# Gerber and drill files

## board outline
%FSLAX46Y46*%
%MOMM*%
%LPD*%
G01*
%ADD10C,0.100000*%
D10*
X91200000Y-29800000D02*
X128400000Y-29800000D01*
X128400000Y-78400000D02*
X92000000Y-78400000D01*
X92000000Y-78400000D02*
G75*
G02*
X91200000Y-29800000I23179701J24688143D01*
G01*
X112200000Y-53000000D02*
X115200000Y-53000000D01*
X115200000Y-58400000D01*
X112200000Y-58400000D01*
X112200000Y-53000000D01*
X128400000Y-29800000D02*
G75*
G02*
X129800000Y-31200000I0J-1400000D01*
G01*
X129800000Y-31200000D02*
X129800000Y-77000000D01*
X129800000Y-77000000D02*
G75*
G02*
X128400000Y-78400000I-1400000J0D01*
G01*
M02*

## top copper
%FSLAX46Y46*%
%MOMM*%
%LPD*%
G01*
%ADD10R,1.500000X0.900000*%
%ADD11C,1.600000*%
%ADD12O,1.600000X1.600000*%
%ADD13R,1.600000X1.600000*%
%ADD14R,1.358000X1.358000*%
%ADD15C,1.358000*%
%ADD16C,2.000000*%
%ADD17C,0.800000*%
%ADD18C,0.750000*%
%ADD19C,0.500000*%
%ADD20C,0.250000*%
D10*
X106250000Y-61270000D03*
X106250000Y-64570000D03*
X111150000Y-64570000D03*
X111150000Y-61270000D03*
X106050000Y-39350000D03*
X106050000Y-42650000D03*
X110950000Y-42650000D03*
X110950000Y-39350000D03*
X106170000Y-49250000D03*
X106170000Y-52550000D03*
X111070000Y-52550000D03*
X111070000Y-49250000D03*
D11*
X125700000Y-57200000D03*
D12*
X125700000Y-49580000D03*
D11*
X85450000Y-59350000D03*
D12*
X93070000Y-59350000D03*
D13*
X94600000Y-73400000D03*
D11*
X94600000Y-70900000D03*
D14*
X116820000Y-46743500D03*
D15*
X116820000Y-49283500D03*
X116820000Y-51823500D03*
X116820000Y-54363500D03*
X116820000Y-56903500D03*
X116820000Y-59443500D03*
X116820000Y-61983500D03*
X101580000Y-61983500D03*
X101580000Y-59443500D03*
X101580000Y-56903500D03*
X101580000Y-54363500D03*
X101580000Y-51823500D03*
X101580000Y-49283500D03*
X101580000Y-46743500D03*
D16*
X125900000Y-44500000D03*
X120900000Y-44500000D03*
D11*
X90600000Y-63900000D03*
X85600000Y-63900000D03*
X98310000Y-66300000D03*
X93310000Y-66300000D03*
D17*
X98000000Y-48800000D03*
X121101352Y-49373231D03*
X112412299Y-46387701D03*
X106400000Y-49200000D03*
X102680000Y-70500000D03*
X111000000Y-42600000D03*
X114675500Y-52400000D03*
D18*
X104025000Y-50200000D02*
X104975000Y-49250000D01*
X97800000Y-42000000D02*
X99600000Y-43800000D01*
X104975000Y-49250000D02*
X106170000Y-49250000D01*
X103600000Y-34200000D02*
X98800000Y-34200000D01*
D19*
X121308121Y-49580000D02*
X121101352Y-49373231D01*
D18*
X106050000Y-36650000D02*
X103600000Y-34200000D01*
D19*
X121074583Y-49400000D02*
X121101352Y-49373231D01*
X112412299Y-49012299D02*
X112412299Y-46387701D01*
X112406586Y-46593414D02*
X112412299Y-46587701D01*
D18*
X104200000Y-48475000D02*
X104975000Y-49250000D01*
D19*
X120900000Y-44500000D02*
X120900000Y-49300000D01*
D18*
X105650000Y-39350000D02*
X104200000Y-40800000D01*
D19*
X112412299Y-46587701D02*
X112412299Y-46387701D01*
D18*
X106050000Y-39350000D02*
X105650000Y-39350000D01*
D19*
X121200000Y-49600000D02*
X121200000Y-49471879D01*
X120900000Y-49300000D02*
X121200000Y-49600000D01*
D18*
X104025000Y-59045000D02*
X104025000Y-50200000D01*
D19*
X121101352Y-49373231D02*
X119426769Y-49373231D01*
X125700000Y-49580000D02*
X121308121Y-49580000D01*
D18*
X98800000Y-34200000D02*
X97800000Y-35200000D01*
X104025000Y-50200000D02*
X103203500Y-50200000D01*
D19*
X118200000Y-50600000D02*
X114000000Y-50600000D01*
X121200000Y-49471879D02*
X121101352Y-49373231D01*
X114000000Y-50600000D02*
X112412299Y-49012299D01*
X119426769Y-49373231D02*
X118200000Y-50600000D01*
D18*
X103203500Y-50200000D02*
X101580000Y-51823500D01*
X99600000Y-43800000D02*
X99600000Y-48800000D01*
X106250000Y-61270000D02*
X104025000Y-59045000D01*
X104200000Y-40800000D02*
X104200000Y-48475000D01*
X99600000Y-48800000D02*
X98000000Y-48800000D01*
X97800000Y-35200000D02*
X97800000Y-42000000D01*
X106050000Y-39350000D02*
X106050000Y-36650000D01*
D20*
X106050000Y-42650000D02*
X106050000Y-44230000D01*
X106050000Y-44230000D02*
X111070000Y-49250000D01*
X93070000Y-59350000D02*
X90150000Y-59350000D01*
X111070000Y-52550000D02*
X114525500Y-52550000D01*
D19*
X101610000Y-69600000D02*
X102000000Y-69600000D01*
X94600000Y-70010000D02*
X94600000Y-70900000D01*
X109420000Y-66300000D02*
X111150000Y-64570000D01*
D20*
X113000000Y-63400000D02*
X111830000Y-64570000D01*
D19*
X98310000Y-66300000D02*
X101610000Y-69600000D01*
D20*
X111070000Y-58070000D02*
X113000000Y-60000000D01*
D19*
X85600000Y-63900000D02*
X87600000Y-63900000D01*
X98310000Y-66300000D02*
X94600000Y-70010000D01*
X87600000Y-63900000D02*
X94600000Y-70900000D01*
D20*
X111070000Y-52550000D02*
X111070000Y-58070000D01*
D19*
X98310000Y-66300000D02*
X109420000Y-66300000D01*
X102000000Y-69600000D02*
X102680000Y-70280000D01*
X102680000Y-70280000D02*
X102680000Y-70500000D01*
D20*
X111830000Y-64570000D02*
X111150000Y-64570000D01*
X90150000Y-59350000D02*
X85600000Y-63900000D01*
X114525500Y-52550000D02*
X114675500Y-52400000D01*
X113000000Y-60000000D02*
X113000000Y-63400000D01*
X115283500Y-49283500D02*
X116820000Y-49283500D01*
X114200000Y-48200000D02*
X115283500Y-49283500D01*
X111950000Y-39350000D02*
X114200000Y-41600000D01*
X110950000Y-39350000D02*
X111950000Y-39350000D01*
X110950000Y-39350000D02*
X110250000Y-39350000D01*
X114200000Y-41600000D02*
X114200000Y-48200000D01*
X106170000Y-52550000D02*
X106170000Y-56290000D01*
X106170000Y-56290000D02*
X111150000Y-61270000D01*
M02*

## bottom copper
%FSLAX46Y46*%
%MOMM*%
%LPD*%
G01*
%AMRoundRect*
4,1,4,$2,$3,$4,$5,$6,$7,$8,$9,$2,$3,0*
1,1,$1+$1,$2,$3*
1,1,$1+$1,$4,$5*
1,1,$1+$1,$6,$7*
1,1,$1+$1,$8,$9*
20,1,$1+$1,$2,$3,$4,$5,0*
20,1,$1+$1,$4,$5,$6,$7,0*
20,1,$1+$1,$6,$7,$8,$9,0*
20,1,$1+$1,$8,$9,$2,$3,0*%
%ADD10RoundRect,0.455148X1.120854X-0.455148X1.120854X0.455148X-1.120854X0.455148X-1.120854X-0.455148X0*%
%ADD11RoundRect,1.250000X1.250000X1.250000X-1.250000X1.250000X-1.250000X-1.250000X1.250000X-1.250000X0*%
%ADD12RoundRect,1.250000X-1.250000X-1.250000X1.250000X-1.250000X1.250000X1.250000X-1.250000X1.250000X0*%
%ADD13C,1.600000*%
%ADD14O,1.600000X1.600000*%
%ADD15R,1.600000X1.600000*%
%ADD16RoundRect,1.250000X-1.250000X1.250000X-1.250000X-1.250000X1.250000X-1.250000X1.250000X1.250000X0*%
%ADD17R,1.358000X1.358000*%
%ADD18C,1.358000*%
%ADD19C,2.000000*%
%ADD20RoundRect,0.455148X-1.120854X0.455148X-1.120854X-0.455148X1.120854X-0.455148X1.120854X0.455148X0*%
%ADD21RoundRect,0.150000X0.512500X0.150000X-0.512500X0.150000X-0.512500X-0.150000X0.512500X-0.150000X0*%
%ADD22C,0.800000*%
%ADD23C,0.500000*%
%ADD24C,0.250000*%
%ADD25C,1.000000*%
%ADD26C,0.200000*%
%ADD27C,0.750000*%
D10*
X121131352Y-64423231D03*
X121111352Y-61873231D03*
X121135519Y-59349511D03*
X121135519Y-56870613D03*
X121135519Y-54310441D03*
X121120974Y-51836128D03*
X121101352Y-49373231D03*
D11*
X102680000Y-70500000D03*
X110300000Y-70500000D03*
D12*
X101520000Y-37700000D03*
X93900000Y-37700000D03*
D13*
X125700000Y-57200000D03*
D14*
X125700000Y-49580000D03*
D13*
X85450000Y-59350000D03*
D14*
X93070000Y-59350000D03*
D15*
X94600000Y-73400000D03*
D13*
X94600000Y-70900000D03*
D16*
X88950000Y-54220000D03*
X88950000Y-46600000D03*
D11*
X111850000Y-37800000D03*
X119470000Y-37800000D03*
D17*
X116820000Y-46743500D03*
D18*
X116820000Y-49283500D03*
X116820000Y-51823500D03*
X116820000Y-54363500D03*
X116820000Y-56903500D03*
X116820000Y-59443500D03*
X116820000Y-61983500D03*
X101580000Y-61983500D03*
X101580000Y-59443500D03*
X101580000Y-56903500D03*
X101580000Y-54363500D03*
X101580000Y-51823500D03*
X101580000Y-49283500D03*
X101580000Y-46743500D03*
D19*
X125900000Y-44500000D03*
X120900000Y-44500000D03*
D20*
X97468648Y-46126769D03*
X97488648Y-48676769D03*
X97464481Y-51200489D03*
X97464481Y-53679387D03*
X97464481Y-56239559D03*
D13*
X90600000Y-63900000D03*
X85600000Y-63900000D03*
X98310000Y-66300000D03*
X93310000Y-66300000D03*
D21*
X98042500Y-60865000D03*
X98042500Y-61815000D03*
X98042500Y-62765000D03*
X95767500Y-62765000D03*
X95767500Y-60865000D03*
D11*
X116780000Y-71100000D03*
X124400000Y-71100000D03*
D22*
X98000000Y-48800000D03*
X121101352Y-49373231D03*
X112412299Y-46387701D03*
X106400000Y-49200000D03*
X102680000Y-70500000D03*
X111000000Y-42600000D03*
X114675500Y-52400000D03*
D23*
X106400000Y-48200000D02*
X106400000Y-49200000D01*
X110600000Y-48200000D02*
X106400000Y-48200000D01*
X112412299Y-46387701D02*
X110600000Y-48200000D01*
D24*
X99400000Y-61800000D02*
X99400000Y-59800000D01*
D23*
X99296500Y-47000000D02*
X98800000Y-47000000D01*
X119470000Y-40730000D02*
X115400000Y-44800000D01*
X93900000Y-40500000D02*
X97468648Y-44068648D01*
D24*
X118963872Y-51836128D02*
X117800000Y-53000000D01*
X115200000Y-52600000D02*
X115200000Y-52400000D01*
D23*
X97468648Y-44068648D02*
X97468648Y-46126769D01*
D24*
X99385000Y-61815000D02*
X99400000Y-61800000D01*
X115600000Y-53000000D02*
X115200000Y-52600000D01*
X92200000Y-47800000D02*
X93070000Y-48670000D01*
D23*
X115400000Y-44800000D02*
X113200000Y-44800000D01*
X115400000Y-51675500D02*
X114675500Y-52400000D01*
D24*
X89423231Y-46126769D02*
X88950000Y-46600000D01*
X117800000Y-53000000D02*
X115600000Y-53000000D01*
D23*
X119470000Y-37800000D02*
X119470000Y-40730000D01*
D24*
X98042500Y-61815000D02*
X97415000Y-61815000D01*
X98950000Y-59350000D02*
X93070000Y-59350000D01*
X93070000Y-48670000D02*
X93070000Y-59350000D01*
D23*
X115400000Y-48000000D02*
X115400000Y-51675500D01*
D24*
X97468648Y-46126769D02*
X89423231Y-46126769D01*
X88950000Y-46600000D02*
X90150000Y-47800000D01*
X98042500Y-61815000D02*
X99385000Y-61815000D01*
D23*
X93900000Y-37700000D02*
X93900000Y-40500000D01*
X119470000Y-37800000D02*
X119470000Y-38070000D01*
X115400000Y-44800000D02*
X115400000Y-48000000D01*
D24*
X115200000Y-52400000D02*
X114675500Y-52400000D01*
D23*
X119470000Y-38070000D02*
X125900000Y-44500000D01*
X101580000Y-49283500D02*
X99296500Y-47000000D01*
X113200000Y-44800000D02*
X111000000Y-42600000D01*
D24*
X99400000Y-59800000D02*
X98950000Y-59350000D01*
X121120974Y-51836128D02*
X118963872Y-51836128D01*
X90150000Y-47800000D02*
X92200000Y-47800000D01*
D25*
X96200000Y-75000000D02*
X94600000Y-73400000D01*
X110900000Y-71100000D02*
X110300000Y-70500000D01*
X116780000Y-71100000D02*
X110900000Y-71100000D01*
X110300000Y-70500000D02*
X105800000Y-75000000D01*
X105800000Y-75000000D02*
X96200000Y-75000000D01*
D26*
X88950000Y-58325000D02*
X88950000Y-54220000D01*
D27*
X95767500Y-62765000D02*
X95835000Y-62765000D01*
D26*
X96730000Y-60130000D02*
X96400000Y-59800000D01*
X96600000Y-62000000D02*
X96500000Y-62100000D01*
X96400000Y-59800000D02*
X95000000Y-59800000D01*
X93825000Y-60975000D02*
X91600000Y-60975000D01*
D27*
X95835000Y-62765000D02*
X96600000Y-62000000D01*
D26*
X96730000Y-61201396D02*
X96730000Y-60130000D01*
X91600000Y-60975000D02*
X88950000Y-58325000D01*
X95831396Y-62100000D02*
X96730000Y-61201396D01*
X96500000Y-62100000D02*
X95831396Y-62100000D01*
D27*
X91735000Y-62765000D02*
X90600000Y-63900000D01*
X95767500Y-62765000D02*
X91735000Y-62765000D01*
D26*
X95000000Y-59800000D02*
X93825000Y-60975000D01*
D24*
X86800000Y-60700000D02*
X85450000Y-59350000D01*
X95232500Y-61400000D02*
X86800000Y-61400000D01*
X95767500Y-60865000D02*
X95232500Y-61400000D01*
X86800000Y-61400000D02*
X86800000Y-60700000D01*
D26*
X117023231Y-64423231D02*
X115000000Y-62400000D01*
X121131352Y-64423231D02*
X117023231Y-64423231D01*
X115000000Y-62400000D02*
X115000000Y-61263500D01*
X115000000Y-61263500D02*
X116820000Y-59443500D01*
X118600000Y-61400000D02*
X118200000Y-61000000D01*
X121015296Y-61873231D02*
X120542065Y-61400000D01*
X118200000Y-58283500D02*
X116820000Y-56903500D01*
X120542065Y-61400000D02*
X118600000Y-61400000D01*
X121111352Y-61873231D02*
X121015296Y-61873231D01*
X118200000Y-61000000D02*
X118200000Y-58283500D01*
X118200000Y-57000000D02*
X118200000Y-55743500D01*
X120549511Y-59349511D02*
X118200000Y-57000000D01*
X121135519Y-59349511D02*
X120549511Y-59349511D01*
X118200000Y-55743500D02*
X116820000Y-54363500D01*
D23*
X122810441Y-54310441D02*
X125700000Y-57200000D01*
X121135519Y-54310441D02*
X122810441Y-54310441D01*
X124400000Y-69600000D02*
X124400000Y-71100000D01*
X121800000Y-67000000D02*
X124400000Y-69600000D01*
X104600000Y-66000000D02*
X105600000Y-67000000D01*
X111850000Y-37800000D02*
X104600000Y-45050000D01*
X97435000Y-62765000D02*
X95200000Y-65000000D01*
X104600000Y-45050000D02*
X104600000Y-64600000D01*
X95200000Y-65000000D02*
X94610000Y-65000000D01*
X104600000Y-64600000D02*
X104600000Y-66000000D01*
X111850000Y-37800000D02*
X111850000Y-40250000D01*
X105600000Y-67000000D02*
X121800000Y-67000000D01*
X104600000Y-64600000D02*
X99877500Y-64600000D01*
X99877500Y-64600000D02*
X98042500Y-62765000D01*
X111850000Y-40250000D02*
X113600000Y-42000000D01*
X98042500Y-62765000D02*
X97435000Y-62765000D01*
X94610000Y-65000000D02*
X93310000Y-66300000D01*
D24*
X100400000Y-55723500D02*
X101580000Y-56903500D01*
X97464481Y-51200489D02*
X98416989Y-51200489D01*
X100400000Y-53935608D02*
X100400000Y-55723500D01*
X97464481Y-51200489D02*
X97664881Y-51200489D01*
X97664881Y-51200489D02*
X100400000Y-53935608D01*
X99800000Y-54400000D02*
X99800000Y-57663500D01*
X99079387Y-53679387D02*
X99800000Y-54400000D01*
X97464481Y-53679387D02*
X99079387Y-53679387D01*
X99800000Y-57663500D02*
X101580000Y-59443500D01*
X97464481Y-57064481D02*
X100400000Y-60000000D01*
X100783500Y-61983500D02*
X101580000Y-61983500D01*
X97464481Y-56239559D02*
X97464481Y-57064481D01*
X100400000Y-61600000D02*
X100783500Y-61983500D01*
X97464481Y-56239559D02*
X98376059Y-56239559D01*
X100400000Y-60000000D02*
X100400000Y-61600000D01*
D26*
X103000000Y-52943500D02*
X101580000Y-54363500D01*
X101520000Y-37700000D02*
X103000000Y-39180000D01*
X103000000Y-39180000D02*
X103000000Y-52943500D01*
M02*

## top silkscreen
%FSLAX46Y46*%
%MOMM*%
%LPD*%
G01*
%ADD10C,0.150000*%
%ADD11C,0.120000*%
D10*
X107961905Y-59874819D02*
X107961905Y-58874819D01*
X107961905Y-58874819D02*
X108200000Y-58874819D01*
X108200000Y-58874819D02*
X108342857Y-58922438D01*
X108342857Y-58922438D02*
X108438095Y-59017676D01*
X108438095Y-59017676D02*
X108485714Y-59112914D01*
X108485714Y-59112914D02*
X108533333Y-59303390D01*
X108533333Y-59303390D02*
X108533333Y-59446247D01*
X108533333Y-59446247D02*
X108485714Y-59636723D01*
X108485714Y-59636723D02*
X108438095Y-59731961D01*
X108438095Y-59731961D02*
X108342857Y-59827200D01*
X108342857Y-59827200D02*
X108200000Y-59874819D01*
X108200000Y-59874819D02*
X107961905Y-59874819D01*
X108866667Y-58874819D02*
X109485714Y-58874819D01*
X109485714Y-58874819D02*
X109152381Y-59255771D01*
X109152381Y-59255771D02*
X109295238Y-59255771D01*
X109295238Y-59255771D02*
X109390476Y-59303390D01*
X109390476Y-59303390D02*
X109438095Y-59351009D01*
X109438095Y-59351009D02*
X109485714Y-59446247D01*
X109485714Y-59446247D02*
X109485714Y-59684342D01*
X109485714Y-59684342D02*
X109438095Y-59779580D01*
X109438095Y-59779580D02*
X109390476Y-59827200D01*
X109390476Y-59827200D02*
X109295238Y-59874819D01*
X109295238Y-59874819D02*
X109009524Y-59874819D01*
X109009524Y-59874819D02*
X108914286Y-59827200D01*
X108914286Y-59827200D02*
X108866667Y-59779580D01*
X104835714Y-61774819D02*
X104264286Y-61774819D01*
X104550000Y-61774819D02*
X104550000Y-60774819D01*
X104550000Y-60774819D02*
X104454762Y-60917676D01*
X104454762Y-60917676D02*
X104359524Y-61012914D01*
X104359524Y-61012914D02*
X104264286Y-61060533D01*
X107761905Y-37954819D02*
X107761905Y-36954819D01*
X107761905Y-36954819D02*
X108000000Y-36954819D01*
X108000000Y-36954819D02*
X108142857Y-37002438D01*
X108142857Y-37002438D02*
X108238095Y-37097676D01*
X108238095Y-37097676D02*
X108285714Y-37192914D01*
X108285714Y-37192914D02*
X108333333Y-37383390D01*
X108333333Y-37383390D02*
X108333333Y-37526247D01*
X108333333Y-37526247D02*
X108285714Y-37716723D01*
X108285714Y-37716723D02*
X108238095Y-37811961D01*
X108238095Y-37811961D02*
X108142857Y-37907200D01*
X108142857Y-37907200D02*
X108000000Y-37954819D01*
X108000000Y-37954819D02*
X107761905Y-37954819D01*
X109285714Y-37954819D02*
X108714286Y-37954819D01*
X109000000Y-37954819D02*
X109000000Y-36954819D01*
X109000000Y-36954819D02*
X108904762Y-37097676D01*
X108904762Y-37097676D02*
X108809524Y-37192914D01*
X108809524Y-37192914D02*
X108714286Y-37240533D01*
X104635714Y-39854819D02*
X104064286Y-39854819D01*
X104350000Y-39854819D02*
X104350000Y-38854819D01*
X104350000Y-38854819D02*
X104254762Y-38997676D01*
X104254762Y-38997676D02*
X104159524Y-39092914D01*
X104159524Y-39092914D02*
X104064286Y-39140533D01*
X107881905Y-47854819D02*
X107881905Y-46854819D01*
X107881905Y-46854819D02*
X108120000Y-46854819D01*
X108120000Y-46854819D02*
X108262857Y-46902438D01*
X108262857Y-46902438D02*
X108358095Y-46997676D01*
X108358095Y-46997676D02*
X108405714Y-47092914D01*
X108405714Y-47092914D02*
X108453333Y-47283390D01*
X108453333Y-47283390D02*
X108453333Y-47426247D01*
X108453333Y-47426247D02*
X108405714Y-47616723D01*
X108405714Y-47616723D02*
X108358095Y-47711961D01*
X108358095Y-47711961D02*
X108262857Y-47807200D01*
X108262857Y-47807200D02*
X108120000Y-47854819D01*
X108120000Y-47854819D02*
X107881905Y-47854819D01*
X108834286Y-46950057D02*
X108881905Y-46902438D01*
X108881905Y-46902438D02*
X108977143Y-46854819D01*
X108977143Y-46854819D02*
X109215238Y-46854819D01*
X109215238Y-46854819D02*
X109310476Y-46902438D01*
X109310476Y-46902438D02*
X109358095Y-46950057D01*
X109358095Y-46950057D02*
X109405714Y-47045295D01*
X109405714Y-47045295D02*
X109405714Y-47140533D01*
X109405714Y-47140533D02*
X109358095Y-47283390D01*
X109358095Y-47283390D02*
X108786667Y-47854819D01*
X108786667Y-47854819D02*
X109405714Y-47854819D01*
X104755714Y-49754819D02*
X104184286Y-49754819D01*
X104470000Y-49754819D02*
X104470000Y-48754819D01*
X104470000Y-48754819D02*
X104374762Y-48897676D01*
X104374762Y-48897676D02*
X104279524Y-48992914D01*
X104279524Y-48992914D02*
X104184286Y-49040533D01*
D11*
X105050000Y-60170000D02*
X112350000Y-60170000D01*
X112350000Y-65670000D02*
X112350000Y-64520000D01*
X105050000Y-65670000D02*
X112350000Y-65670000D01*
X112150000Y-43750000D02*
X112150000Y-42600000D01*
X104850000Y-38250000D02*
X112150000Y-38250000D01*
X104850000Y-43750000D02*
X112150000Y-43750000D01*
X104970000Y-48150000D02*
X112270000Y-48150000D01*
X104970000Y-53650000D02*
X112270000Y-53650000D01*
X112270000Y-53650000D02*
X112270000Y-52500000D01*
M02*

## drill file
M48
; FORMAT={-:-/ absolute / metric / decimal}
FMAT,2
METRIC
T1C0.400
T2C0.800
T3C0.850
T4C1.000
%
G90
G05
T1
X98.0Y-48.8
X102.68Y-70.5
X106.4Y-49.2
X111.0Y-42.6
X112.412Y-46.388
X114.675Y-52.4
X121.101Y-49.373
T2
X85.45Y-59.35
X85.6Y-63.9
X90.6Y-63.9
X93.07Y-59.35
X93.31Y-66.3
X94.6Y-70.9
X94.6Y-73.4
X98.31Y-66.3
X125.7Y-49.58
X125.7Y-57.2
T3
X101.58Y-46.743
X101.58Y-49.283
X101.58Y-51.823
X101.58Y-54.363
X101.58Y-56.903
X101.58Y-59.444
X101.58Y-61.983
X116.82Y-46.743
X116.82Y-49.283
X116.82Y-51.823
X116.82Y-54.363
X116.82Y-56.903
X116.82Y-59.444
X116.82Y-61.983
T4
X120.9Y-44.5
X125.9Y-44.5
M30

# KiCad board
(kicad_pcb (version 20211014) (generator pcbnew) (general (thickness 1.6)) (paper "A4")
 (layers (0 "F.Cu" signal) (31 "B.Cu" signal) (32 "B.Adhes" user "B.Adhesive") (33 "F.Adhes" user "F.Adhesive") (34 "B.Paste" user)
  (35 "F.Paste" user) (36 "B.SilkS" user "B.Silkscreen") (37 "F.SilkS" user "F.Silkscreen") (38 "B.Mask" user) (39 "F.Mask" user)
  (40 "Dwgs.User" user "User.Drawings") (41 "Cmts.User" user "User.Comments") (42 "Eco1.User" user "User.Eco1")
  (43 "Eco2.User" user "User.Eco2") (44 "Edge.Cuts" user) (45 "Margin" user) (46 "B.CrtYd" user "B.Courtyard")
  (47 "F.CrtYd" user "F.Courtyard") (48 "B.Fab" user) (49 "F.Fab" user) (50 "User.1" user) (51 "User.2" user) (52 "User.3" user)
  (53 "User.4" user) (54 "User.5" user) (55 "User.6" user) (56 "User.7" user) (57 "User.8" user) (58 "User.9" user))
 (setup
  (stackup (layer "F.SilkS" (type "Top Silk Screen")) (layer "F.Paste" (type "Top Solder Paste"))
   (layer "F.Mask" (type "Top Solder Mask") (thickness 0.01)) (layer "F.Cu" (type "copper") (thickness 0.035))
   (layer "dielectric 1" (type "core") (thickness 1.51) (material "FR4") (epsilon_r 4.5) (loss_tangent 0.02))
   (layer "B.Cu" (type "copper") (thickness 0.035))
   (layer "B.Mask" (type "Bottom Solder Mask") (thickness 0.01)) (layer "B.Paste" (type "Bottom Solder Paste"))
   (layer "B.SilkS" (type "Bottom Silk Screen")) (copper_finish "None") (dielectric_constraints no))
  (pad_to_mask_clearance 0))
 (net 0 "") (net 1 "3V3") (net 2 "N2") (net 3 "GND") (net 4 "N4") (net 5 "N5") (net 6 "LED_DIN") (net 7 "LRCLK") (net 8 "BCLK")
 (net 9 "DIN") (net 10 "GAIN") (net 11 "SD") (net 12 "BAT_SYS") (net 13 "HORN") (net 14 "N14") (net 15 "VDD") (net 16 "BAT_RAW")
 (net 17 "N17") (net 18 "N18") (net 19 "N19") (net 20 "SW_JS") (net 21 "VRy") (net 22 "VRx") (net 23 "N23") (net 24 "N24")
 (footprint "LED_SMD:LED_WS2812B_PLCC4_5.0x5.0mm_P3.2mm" (layer "F.Cu") (at 108.7 62.92)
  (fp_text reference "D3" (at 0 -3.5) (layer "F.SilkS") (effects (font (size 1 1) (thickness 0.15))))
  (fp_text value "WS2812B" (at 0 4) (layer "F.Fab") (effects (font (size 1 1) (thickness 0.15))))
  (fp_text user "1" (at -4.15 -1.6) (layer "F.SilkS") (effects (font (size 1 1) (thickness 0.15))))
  (fp_line (start -3.65 -2.75) (end 3.65 -2.75) (layer "F.SilkS") (width 0.12))
  (fp_line (start 3.65 2.75) (end 3.65 1.6) (layer "F.SilkS") (width 0.12))
  (fp_line (start -3.65 2.75) (end 3.65 2.75) (layer "F.SilkS") (width 0.12))
  (pad "1" smd rect (at -2.45 -1.65) (size 1.5 0.9) (layers "F.Cu" "F.Paste" "F.Mask") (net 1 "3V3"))
  (pad "2" smd rect (at -2.45 1.65) (size 1.5 0.9) (layers "F.Cu" "F.Paste" "F.Mask") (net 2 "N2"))
  (pad "3" smd rect (at 2.45 1.65) (size 1.5 0.9) (layers "F.Cu" "F.Paste" "F.Mask") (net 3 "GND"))
  (pad "4" smd rect (at 2.45 -1.65) (size 1.5 0.9) (layers "F.Cu" "F.Paste" "F.Mask") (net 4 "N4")))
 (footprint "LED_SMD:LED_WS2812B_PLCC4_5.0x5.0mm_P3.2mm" (layer "F.Cu") (at 108.5 41)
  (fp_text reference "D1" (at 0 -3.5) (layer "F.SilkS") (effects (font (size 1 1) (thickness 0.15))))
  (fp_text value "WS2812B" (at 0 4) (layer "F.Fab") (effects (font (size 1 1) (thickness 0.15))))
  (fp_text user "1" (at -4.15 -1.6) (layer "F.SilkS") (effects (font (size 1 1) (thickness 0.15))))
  (fp_line (start 3.65 2.75) (end 3.65 1.6) (layer "F.SilkS") (width 0.12))
  (fp_line (start -3.65 -2.75) (end 3.65 -2.75) (layer "F.SilkS") (width 0.12))
  (fp_line (start -3.65 2.75) (end 3.65 2.75) (layer "F.SilkS") (width 0.12))
  (pad "1" smd rect (at -2.45 -1.65) (size 1.5 0.9) (layers "F.Cu" "F.Paste" "F.Mask") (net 1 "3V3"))
  (pad "2" smd rect (at -2.45 1.65) (size 1.5 0.9) (layers "F.Cu" "F.Paste" "F.Mask") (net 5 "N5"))
  (pad "3" smd rect (at 2.45 1.65) (size 1.5 0.9) (layers "F.Cu" "F.Paste" "F.Mask") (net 3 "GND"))
  (pad "4" smd rect (at 2.45 -1.65) (size 1.5 0.9) (layers "F.Cu" "F.Paste" "F.Mask") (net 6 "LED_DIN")))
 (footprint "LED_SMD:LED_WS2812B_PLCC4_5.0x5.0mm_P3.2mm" (layer "F.Cu") (at 108.62 50.9)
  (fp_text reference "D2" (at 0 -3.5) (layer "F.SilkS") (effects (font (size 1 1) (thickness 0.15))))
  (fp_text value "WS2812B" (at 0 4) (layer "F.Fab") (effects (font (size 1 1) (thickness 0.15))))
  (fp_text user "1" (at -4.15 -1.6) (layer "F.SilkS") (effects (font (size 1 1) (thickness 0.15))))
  (fp_line (start -3.65 -2.75) (end 3.65 -2.75) (layer "F.SilkS") (width 0.12))
  (fp_line (start -3.65 2.75) (end 3.65 2.75) (layer "F.SilkS") (width 0.12))
  (fp_line (start 3.65 2.75) (end 3.65 1.6) (layer "F.SilkS") (width 0.12))
  (pad "1" smd rect (at -2.45 -1.65) (size 1.5 0.9) (layers "F.Cu" "F.Paste" "F.Mask") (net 1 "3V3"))
  (pad "2" smd rect (at -2.45 1.65) (size 1.5 0.9) (layers "F.Cu" "F.Paste" "F.Mask") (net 4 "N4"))
  (pad "3" smd rect (at 2.45 1.65) (size 1.5 0.9) (layers "F.Cu" "F.Paste" "F.Mask") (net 3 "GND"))
  (pad "4" smd rect (at 2.45 -1.65) (size 1.5 0.9) (layers "F.Cu" "F.Paste" "F.Mask") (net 5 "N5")))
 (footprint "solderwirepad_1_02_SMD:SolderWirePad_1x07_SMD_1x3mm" (layer "B.Cu") (at 121.1 64.4 90)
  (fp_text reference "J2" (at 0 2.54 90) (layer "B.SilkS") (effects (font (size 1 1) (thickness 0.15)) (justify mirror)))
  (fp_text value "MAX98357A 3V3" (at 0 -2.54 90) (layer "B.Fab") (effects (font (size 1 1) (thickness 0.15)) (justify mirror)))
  (pad "1" smd roundrect (at -0.023231 0.031352 90) (size 1.820592 3.152005) (layers "B.Cu" "B.Paste" "B.Mask") (roundrect_rratio 0.25)
   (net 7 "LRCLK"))
  (pad "2" smd roundrect (at 2.526769 0.011352 90) (size 1.820592 3.152005) (layers "B.Cu" "B.Paste" "B.Mask") (roundrect_rratio 0.25)
   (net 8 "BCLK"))
  (pad "3" smd roundrect (at 5.050489 0.035519 90) (size 1.820592 3.152005) (layers "B.Cu" "B.Paste" "B.Mask") (roundrect_rratio 0.25)
   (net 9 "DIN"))
  (pad "4" smd roundrect (at 7.529387 0.035519 90) (size 1.820592 3.152005) (layers "B.Cu" "B.Paste" "B.Mask") (roundrect_rratio 0.25)
   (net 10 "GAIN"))
  (pad "5" smd roundrect (at 10.089559 0.035519 90) (size 1.820592 3.152005) (layers "B.Cu" "B.Paste" "B.Mask") (roundrect_rratio 0.25)
   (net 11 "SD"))
  (pad "6" smd roundrect (at 12.563872 0.020974 90) (size 1.820592 3.152005) (layers "B.Cu" "B.Paste" "B.Mask") (roundrect_rratio 0.25)
   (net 3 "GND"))
  (pad "7" smd roundrect (at 15.026769 0.001352 90) (size 1.820592 3.152005) (layers "B.Cu" "B.Paste" "B.Mask") (roundrect_rratio 0.25)
   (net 1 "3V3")))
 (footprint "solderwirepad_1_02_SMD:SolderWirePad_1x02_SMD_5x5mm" (layer "B.Cu") (at 110.3 70.5 180)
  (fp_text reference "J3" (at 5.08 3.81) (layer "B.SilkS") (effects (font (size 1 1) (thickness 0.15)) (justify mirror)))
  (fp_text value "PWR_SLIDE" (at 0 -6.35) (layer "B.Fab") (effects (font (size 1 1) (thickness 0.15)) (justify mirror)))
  (pad "1" smd roundrect (at 7.62 0 180) (size 5 5) (layers "B.Cu" "B.Paste" "B.Mask") (roundrect_rratio 0.25) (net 3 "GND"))
  (pad "2" smd roundrect (at 0 0 180) (size 5 5) (layers "B.Cu" "B.Paste" "B.Mask") (roundrect_rratio 0.25) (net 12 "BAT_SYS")))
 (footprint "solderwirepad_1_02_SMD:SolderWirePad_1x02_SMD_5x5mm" (layer "B.Cu") (at 93.9 37.7)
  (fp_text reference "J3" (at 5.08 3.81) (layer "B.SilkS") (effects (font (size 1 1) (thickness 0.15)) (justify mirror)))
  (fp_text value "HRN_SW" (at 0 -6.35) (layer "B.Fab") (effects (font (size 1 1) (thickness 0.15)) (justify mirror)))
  (pad "1" smd roundrect (at 7.62 0) (size 5 5) (layers "B.Cu" "B.Paste" "B.Mask") (roundrect_rratio 0.25) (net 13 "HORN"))
  (pad "2" smd roundrect (at 0 0) (size 5 5) (layers "B.Cu" "B.Paste" "B.Mask") (roundrect_rratio 0.25) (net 3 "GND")))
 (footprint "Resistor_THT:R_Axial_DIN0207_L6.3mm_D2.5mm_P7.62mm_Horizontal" (layer "B.Cu") (at 125.7 57.2 90)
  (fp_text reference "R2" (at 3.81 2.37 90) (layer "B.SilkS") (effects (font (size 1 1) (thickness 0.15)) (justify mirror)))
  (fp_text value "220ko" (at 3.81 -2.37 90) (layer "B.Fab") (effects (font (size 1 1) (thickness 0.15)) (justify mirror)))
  (pad "1" thru_hole circle (at 0 0 90) (size 1.6 1.6) (drill 0.8) (layers *.Cu *.Mask) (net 11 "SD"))
  (pad "2" thru_hole oval (at 7.62 0 90) (size 1.6 1.6) (drill 0.8) (layers *.Cu *.Mask) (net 1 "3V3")))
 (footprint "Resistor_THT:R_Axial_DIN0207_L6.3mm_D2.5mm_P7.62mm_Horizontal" (layer "B.Cu") (at 85.45 59.35)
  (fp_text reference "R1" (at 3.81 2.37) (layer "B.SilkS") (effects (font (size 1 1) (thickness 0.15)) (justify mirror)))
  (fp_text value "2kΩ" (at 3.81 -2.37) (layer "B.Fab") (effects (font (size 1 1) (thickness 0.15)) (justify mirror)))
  (pad "1" thru_hole circle (at 0 0) (size 1.6 1.6) (drill 0.8) (layers *.Cu *.Mask) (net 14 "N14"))
  (pad "2" thru_hole oval (at 7.62 0) (size 1.6 1.6) (drill 0.8) (layers *.Cu *.Mask) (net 3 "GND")))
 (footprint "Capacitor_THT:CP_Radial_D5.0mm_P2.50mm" (layer "B.Cu") (at 94.6 73.4 90)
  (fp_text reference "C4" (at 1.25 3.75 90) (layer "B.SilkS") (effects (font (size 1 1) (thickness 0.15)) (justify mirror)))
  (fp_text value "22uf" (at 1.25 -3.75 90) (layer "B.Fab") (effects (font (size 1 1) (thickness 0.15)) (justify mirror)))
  (pad "1" thru_hole rect (at 0 0 90) (size 1.6 1.6) (drill 0.8) (layers *.Cu *.Mask) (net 12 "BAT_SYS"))
  (pad "2" thru_hole circle (at 2.5 0 90) (size 1.6 1.6) (drill 0.8) (layers *.Cu *.Mask) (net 3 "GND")))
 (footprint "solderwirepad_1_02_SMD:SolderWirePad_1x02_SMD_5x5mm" (layer "B.Cu") (at 88.95 46.6 -90)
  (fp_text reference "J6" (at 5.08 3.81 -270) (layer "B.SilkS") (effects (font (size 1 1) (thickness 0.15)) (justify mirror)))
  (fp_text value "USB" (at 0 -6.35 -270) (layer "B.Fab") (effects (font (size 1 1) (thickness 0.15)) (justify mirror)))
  (pad "1" smd roundrect (at 7.62 0 270) (size 5 5) (layers "B.Cu" "B.Paste" "B.Mask") (roundrect_rratio 0.25) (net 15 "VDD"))
  (pad "2" smd roundrect (at 0 0 270) (size 5 5) (layers "B.Cu" "B.Paste" "B.Mask") (roundrect_rratio 0.25) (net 3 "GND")))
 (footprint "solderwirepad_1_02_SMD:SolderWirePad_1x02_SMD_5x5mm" (layer "B.Cu") (at 119.47 37.8 180)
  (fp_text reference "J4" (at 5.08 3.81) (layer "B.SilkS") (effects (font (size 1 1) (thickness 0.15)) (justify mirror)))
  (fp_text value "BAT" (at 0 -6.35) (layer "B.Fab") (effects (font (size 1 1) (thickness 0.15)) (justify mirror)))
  (pad "1" smd roundrect (at 7.62 0 180) (size 5 5) (layers "B.Cu" "B.Paste" "B.Mask") (roundrect_rratio 0.25) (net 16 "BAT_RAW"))
  (pad "2" smd roundrect (at 0 0 180) (size 5 5) (layers "B.Cu" "B.Paste" "B.Mask") (roundrect_rratio 0.25) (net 3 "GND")))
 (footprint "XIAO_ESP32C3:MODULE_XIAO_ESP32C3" (layer "B.Cu") (at 109.2 54.3 180)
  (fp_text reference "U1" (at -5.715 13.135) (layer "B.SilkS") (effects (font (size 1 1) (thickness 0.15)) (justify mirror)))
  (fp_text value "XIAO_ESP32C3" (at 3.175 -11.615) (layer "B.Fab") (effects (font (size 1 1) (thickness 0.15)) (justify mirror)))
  (pad "1" thru_hole rect (at -7.62 7.5565 180) (size 1.358 1.358) (drill 0.85) (layers *.Cu *.Mask) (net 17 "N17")
   (solder_mask_margin 0.102))
  (pad "2" thru_hole circle (at -7.62 5.0165 180) (size 1.358 1.358) (drill 0.85) (layers *.Cu *.Mask) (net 6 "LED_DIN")
   (solder_mask_margin 0.102))
  (pad "3" thru_hole circle (at -7.62 2.4765 180) (size 1.358 1.358) (drill 0.85) (layers *.Cu *.Mask) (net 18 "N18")
   (solder_mask_margin 0.102))
  (pad "4" thru_hole circle (at -7.62 -0.0635 180) (size 1.358 1.358) (drill 0.85) (layers *.Cu *.Mask) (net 9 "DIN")
   (solder_mask_margin 0.102))
  (pad "5" thru_hole circle (at -7.62 -2.6035 180) (size 1.358 1.358) (drill 0.85) (layers *.Cu *.Mask) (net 8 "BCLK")
   (solder_mask_margin 0.102))
  (pad "6" thru_hole circle (at -7.62 -5.1435 180) (size 1.358 1.358) (drill 0.85) (layers *.Cu *.Mask) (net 7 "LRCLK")
   (solder_mask_margin 0.102))
  (pad "7" thru_hole circle (at -7.62 -7.6835 180) (size 1.358 1.358) (drill 0.85) (layers *.Cu *.Mask) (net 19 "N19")
   (solder_mask_margin 0.102))
  (pad "8" thru_hole circle (at 7.62 -7.6835 180) (size 1.358 1.358) (drill 0.85) (layers *.Cu *.Mask) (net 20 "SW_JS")
   (solder_mask_margin 0.102))
  (pad "9" thru_hole circle (at 7.62 -5.1435 180) (size 1.358 1.358) (drill 0.85) (layers *.Cu *.Mask) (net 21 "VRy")
   (solder_mask_margin 0.102))
  (pad "10" thru_hole circle (at 7.62 -2.6035 180) (size 1.358 1.358) (drill 0.85) (layers *.Cu *.Mask) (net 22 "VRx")
   (solder_mask_margin 0.102))
  (pad "11" thru_hole circle (at 7.62 -0.0635 180) (size 1.358 1.358) (drill 0.85) (layers *.Cu *.Mask) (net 13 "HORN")
   (solder_mask_margin 0.102))
  (pad "12" thru_hole circle (at 7.62 2.4765 180) (size 1.358 1.358) (drill 0.85) (layers *.Cu *.Mask) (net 1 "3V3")
   (solder_mask_margin 0.102))
  (pad "13" thru_hole circle (at 7.62 5.0165 180) (size 1.358 1.358) (drill 0.85) (layers *.Cu *.Mask) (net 3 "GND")
   (solder_mask_margin 0.102))
  (pad "14" thru_hole circle (at 7.62 7.5565 180) (size 1.358 1.358) (drill 0.85) (layers *.Cu *.Mask) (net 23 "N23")
   (solder_mask_margin 0.102)))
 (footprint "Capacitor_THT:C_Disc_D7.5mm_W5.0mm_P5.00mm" (layer "B.Cu") (at 125.9 44.5 180)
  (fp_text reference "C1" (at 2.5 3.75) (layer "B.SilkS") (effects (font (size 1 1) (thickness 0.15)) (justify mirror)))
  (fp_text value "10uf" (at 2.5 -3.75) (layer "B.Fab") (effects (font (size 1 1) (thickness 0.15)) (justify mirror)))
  (pad "1" thru_hole circle (at 0 0 180) (size 2 2) (drill 1) (layers *.Cu *.Mask) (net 3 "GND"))
  (pad "2" thru_hole circle (at 5 0 180) (size 2 2) (drill 1) (layers *.Cu *.Mask) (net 1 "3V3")))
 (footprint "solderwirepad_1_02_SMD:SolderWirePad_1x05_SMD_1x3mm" (layer "B.Cu") (at 97.5 46.15 -90)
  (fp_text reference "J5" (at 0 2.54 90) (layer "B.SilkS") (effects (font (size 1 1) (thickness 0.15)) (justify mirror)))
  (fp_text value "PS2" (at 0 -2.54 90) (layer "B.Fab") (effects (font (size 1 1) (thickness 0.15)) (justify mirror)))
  (pad "1" smd roundrect (at -0.023231 0.031352 270) (size 1.820592 3.152005) (layers "B.Cu" "B.Paste" "B.Mask") (roundrect_rratio 0.25)
   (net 3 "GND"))
  (pad "2" smd roundrect (at 2.526769 0.011352 270) (size 1.820592 3.152005) (layers "B.Cu" "B.Paste" "B.Mask") (roundrect_rratio 0.25)
   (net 1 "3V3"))
  (pad "3" smd roundrect (at 5.050489 0.035519 270) (size 1.820592 3.152005) (layers "B.Cu" "B.Paste" "B.Mask") (roundrect_rratio 0.25)
   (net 22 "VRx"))
  (pad "4" smd roundrect (at 7.529387 0.035519 270) (size 1.820592 3.152005) (layers "B.Cu" "B.Paste" "B.Mask") (roundrect_rratio 0.25)
   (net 21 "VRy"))
  (pad "5" smd roundrect (at 10.089559 0.035519 270) (size 1.820592 3.152005) (layers "B.Cu" "B.Paste" "B.Mask") (roundrect_rratio 0.25)
   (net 20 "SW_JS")))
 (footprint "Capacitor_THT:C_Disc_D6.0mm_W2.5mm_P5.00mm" (layer "B.Cu") (at 90.6 63.9 180)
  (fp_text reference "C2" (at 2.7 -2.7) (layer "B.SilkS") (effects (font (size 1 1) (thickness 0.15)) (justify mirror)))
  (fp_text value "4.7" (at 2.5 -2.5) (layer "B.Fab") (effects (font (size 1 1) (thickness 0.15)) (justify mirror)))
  (pad "1" thru_hole circle (at 0 0 180) (size 1.6 1.6) (drill 0.8) (layers *.Cu *.Mask) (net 15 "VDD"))
  (pad "2" thru_hole circle (at 5 0 180) (size 1.6 1.6) (drill 0.8) (layers *.Cu *.Mask) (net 3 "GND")))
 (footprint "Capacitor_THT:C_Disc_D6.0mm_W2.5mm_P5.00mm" (layer "B.Cu") (at 98.31 66.3 180)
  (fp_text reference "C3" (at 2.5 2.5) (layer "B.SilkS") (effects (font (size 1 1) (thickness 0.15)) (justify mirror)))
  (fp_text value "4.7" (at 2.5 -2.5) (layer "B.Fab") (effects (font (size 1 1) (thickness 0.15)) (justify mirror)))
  (pad "1" thru_hole circle (at 0 0 180) (size 1.6 1.6) (drill 0.8) (layers *.Cu *.Mask) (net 3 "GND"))
  (pad "2" thru_hole circle (at 5 0 180) (size 1.6 1.6) (drill 0.8) (layers *.Cu *.Mask) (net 16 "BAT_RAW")))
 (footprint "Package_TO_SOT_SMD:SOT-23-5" (layer "B.Cu") (at 96.905 61.815 180)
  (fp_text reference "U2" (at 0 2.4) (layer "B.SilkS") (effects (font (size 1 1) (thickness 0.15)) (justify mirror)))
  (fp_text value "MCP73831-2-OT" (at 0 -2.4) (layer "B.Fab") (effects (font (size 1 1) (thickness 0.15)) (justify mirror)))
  (pad "1" smd roundrect (at -1.1375 0.95 180) (size 1.325 0.6) (layers "B.Cu" "B.Paste" "B.Mask") (roundrect_rratio 0.25) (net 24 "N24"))
  (pad "2" smd roundrect (at -1.1375 0 180) (size 1.325 0.6) (layers "B.Cu" "B.Paste" "B.Mask") (roundrect_rratio 0.25) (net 3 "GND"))
  (pad "3" smd roundrect (at -1.1375 -0.95 180) (size 1.325 0.6) (layers "B.Cu" "B.Paste" "B.Mask") (roundrect_rratio 0.25)
   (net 16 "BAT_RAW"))
  (pad "4" smd roundrect (at 1.1375 -0.95 180) (size 1.325 0.6) (layers "B.Cu" "B.Paste" "B.Mask") (roundrect_rratio 0.25) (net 15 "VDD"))
  (pad "5" smd roundrect (at 1.1375 0.95 180) (size 1.325 0.6) (layers "B.Cu" "B.Paste" "B.Mask") (roundrect_rratio 0.25) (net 14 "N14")))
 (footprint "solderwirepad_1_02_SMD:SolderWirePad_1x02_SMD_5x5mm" (layer "B.Cu") (at 124.4 71.1 180)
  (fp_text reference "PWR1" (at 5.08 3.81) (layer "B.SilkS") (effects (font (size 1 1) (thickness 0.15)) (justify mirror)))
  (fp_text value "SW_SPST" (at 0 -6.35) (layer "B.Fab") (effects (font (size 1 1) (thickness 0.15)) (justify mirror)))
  (pad "1" smd roundrect (at 7.62 0 180) (size 5 5) (layers "B.Cu" "B.Paste" "B.Mask") (roundrect_rratio 0.25) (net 12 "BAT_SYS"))
  (pad "2" smd roundrect (at 0 0 180) (size 5 5) (layers "B.Cu" "B.Paste" "B.Mask") (roundrect_rratio 0.25) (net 16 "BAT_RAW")))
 (gr_line (start 91.2 29.8) (end 128.4 29.8) (layer "Edge.Cuts") (width 0.1))
 (gr_line (start 128.4 78.4) (end 92 78.4) (layer "Edge.Cuts") (width 0.1))
 (gr_arc (start 92 78.4) (mid 81.319809 54.269224) (end 91.2 29.8) (layer "Edge.Cuts") (width 0.1))
 (gr_rect (start 112.2 53) (end 115.2 58.4) (layer "Edge.Cuts") (width 0.1) (fill none))
 (gr_arc (start 128.4 29.8) (mid 129.389949 30.210051) (end 129.8 31.2) (layer "Edge.Cuts") (width 0.1))
 (gr_line (start 129.8 31.2) (end 129.8 77) (layer "Edge.Cuts") (width 0.1))
 (gr_arc (start 129.8 77) (mid 129.389949 77.989949) (end 128.4 78.4) (layer "Edge.Cuts") (width 0.1))
 (segment (start 104.025 50.2) (end 104.975 49.25) (width 0.75) (layer "F.Cu") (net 1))
 (segment (start 97.8 42) (end 99.6 43.8) (width 0.75) (layer "F.Cu") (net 1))
 (segment (start 104.975 49.25) (end 106.17 49.25) (width 0.75) (layer "F.Cu") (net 1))
 (segment (start 103.6 34.2) (end 98.8 34.2) (width 0.75) (layer "F.Cu") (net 1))
 (segment (start 121.308121 49.58) (end 121.101352 49.373231) (width 0.5) (layer "F.Cu") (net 1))
 (segment (start 106.05 36.65) (end 103.6 34.2) (width 0.75) (layer "F.Cu") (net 1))
 (segment (start 121.074583 49.4) (end 121.101352 49.373231) (width 0.5) (layer "F.Cu") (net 1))
 (segment (start 112.412299 49.012299) (end 112.412299 46.387701) (width 0.5) (layer "F.Cu") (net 1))
 (segment (start 112.406586 46.593414) (end 112.412299 46.587701) (width 0.5) (layer "F.Cu") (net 1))
 (segment (start 104.2 48.475) (end 104.975 49.25) (width 0.75) (layer "F.Cu") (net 1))
 (segment (start 120.9 44.5) (end 120.9 49.3) (width 0.5) (layer "F.Cu") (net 1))
 (segment (start 105.65 39.35) (end 104.2 40.8) (width 0.75) (layer "F.Cu") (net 1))
 (segment (start 112.412299 46.587701) (end 112.412299 46.387701) (width 0.5) (layer "F.Cu") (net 1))
 (segment (start 106.05 39.35) (end 105.65 39.35) (width 0.75) (layer "F.Cu") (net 1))
 (segment (start 121.2 49.6) (end 121.2 49.471879) (width 0.5) (layer "F.Cu") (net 1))
 (segment (start 120.9 49.3) (end 121.2 49.6) (width 0.5) (layer "F.Cu") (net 1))
 (segment (start 104.025 59.045) (end 104.025 50.2) (width 0.75) (layer "F.Cu") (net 1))
 (segment (start 121.101352 49.373231) (end 119.426769 49.373231) (width 0.5) (layer "F.Cu") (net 1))
 (segment (start 125.7 49.58) (end 121.308121 49.58) (width 0.5) (layer "F.Cu") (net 1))
 (segment (start 98.8 34.2) (end 97.8 35.2) (width 0.75) (layer "F.Cu") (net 1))
 (segment (start 104.025 50.2) (end 103.2035 50.2) (width 0.75) (layer "F.Cu") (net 1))
 (segment (start 118.2 50.6) (end 114 50.6) (width 0.5) (layer "F.Cu") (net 1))
 (segment (start 121.2 49.471879) (end 121.101352 49.373231) (width 0.5) (layer "F.Cu") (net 1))
 (segment (start 114 50.6) (end 112.412299 49.012299) (width 0.5) (layer "F.Cu") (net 1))
 (segment (start 119.426769 49.373231) (end 118.2 50.6) (width 0.5) (layer "F.Cu") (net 1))
 (segment (start 103.2035 50.2) (end 101.58 51.8235) (width 0.75) (layer "F.Cu") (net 1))
 (segment (start 99.6 43.8) (end 99.6 48.8) (width 0.75) (layer "F.Cu") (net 1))
 (segment (start 106.25 61.27) (end 104.025 59.045) (width 0.75) (layer "F.Cu") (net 1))
 (segment (start 104.2 40.8) (end 104.2 48.475) (width 0.75) (layer "F.Cu") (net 1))
 (segment (start 99.6 48.8) (end 98 48.8) (width 0.75) (layer "F.Cu") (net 1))
 (segment (start 97.8 35.2) (end 97.8 42) (width 0.75) (layer "F.Cu") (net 1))
 (segment (start 106.05 39.35) (end 106.05 36.65) (width 0.75) (layer "F.Cu") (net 1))
 (via (at 98 48.8) (size 0.8) (drill 0.4) (layers "F.Cu" "B.Cu") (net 1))
 (via (at 121.101352 49.373231) (size 0.8) (drill 0.4) (layers "F.Cu" "B.Cu") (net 1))
 (via (at 112.412299 46.387701) (size 0.8) (drill 0.4) (layers "F.Cu" "B.Cu") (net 1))
 (via (at 106.4 49.2) (size 0.8) (drill 0.4) (layers "F.Cu" "B.Cu") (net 1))
 (segment (start 106.4 48.2) (end 106.4 49.2) (width 0.5) (layer "B.Cu") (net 1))
 (segment (start 110.6 48.2) (end 106.4 48.2) (width 0.5) (layer "B.Cu") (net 1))
 (segment (start 112.412299 46.387701) (end 110.6 48.2) (width 0.5) (layer "B.Cu") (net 1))
 (segment (start 106.05 42.65) (end 106.05 44.23) (width 0.25) (layer "F.Cu") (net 5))
 (segment (start 106.05 44.23) (end 111.07 49.25) (width 0.25) (layer "F.Cu") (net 5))
 (segment (start 93.07 59.35) (end 90.15 59.35) (width 0.25) (layer "F.Cu") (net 3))
 (segment (start 111.07 52.55) (end 114.5255 52.55) (width 0.25) (layer "F.Cu") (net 3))
 (segment (start 101.61 69.6) (end 102 69.6) (width 0.5) (layer "F.Cu") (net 3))
 (segment (start 94.6 70.01) (end 94.6 70.9) (width 0.5) (layer "F.Cu") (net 3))
 (segment (start 109.42 66.3) (end 111.15 64.57) (width 0.5) (layer "F.Cu") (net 3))
 (segment (start 113 63.4) (end 111.83 64.57) (width 0.25) (layer "F.Cu") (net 3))
 (segment (start 98.31 66.3) (end 101.61 69.6) (width 0.5) (layer "F.Cu") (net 3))
 (segment (start 111.07 58.07) (end 113 60) (width 0.25) (layer "F.Cu") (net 3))
 (segment (start 85.6 63.9) (end 87.6 63.9) (width 0.5) (layer "F.Cu") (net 3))
 (segment (start 98.31 66.3) (end 94.6 70.01) (width 0.5) (layer "F.Cu") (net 3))
 (segment (start 87.6 63.9) (end 94.6 70.9) (width 0.5) (layer "F.Cu") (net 3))
 (segment (start 111.07 52.55) (end 111.07 58.07) (width 0.25) (layer "F.Cu") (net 3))
 (segment (start 98.31 66.3) (end 109.42 66.3) (width 0.5) (layer "F.Cu") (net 3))
 (segment (start 102 69.6) (end 102.68 70.28) (width 0.5) (layer "F.Cu") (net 3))
 (segment (start 102.68 70.28) (end 102.68 70.5) (width 0.5) (layer "F.Cu") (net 3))
 (segment (start 111.83 64.57) (end 111.15 64.57) (width 0.25) (layer "F.Cu") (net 3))
 (segment (start 90.15 59.35) (end 85.6 63.9) (width 0.25) (layer "F.Cu") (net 3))
 (segment (start 114.5255 52.55) (end 114.6755 52.4) (width 0.25) (layer "F.Cu") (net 3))
 (segment (start 113 60) (end 113 63.4) (width 0.25) (layer "F.Cu") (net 3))
 (via (at 102.68 70.5) (size 0.8) (drill 0.4) (layers "F.Cu" "B.Cu") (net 3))
 (via (at 111 42.6) (size 0.8) (drill 0.4) (layers "F.Cu" "B.Cu") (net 3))
 (via (at 114.6755 52.4) (size 0.8) (drill 0.4) (layers "F.Cu" "B.Cu") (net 3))
 (segment (start 99.4 61.8) (end 99.4 59.8) (width 0.25) (layer "B.Cu") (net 3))
 (segment (start 99.2965 47) (end 98.8 47) (width 0.5) (layer "B.Cu") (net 3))
 (segment (start 119.47 40.73) (end 115.4 44.8) (width 0.5) (layer "B.Cu") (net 3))
 (segment (start 93.9 40.5) (end 97.468648 44.068648) (width 0.5) (layer "B.Cu") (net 3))
 (segment (start 118.963872 51.836128) (end 117.8 53) (width 0.25) (layer "B.Cu") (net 3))
 (segment (start 115.2 52.6) (end 115.2 52.4) (width 0.25) (layer "B.Cu") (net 3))
 (segment (start 97.468648 44.068648) (end 97.468648 46.126769) (width 0.5) (layer "B.Cu") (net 3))
 (segment (start 99.385 61.815) (end 99.4 61.8) (width 0.25) (layer "B.Cu") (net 3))
 (segment (start 115.6 53) (end 115.2 52.6) (width 0.25) (layer "B.Cu") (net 3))
 (segment (start 92.2 47.8) (end 93.07 48.67) (width 0.25) (layer "B.Cu") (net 3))
 (segment (start 115.4 44.8) (end 113.2 44.8) (width 0.5) (layer "B.Cu") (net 3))
 (segment (start 115.4 51.6755) (end 114.6755 52.4) (width 0.5) (layer "B.Cu") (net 3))
 (segment (start 89.423231 46.126769) (end 88.95 46.6) (width 0.25) (layer "B.Cu") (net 3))
 (segment (start 117.8 53) (end 115.6 53) (width 0.25) (layer "B.Cu") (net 3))
 (segment (start 119.47 37.8) (end 119.47 40.73) (width 0.5) (layer "B.Cu") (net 3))
 (segment (start 98.0425 61.815) (end 97.415 61.815) (width 0.25) (layer "B.Cu") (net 3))
 (segment (start 98.95 59.35) (end 93.07 59.35) (width 0.25) (layer "B.Cu") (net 3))
 (segment (start 93.07 48.67) (end 93.07 59.35) (width 0.25) (layer "B.Cu") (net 3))
 (segment (start 115.4 48) (end 115.4 51.6755) (width 0.5) (layer "B.Cu") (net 3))
 (segment (start 97.468648 46.126769) (end 89.423231 46.126769) (width 0.25) (layer "B.Cu") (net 3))
 (segment (start 88.95 46.6) (end 90.15 47.8) (width 0.25) (layer "B.Cu") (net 3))
 (segment (start 98.0425 61.815) (end 99.385 61.815) (width 0.25) (layer "B.Cu") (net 3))
 (segment (start 93.9 37.7) (end 93.9 40.5) (width 0.5) (layer "B.Cu") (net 3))
 (segment (start 119.47 37.8) (end 119.47 38.07) (width 0.5) (layer "B.Cu") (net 3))
 (segment (start 115.4 44.8) (end 115.4 48) (width 0.5) (layer "B.Cu") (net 3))
 (segment (start 115.2 52.4) (end 114.6755 52.4) (width 0.25) (layer "B.Cu") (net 3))
 (segment (start 119.47 38.07) (end 125.9 44.5) (width 0.5) (layer "B.Cu") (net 3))
 (segment (start 101.58 49.2835) (end 99.2965 47) (width 0.5) (layer "B.Cu") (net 3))
 (segment (start 113.2 44.8) (end 111 42.6) (width 0.5) (layer "B.Cu") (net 3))
 (segment (start 99.4 59.8) (end 98.95 59.35) (width 0.25) (layer "B.Cu") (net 3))
 (segment (start 121.120974 51.836128) (end 118.963872 51.836128) (width 0.25) (layer "B.Cu") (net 3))
 (segment (start 90.15 47.8) (end 92.2 47.8) (width 0.25) (layer "B.Cu") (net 3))
 (segment (start 115.2835 49.2835) (end 116.82 49.2835) (width 0.25) (layer "F.Cu") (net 6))
 (segment (start 114.2 48.2) (end 115.2835 49.2835) (width 0.25) (layer "F.Cu") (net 6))
 (segment (start 111.95 39.35) (end 114.2 41.6) (width 0.25) (layer "F.Cu") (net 6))
 (segment (start 110.95 39.35) (end 111.95 39.35) (width 0.25) (layer "F.Cu") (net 6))
 (segment (start 110.95 39.35) (end 110.25 39.35) (width 0.25) (layer "F.Cu") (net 6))
 (segment (start 114.2 41.6) (end 114.2 48.2) (width 0.25) (layer "F.Cu") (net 6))
 (segment (start 106.17 52.55) (end 106.17 56.29) (width 0.25) (layer "F.Cu") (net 4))
 (segment (start 106.17 56.29) (end 111.15 61.27) (width 0.25) (layer "F.Cu") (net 4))
 (segment (start 96.2 75) (end 94.6 73.4) (width 1) (layer "B.Cu") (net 12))
 (segment (start 110.9 71.1) (end 110.3 70.5) (width 1) (layer "B.Cu") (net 12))
 (segment (start 116.78 71.1) (end 110.9 71.1) (width 1) (layer "B.Cu") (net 12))
 (segment (start 110.3 70.5) (end 105.8 75) (width 1) (layer "B.Cu") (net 12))
 (segment (start 105.8 75) (end 96.2 75) (width 1) (layer "B.Cu") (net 12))
 (segment (start 88.95 58.325) (end 88.95 54.22) (width 0.2) (layer "B.Cu") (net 15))
 (segment (start 95.7675 62.765) (end 95.835 62.765) (width 0.75) (layer "B.Cu") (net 15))
 (segment (start 96.73 60.13) (end 96.4 59.8) (width 0.2) (layer "B.Cu") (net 15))
 (segment (start 96.6 62) (end 96.5 62.1) (width 0.2) (layer "B.Cu") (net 15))
 (segment (start 96.4 59.8) (end 95 59.8) (width 0.2) (layer "B.Cu") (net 15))
 (segment (start 93.825 60.975) (end 91.6 60.975) (width 0.2) (layer "B.Cu") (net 15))
 (segment (start 95.835 62.765) (end 96.6 62) (width 0.75) (layer "B.Cu") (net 15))
 (segment (start 96.73 61.201396) (end 96.73 60.13) (width 0.2) (layer "B.Cu") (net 15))
 (segment (start 91.6 60.975) (end 88.95 58.325) (width 0.2) (layer "B.Cu") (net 15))
 (segment (start 95.831396 62.1) (end 96.73 61.201396) (width 0.2) (layer "B.Cu") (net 15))
 (segment (start 96.5 62.1) (end 95.831396 62.1) (width 0.2) (layer "B.Cu") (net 15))
 (segment (start 91.735 62.765) (end 90.6 63.9) (width 0.75) (layer "B.Cu") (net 15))
 (segment (start 95.7675 62.765) (end 91.735 62.765) (width 0.75) (layer "B.Cu") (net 15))
 (segment (start 95 59.8) (end 93.825 60.975) (width 0.2) (layer "B.Cu") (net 15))
 (segment (start 86.8 60.7) (end 85.45 59.35) (width 0.25) (layer "B.Cu") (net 14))
 (segment (start 95.2325 61.4) (end 86.8 61.4) (width 0.25) (layer "B.Cu") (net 14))
 (segment (start 95.7675 60.865) (end 95.2325 61.4) (width 0.25) (layer "B.Cu") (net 14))
 (segment (start 86.8 61.4) (end 86.8 60.7) (width 0.25) (layer "B.Cu") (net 14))
 (segment (start 117.023231 64.423231) (end 115 62.4) (width 0.2) (layer "B.Cu") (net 7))
 (segment (start 121.131352 64.423231) (end 117.023231 64.423231) (width 0.2) (layer "B.Cu") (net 7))
 (segment (start 115 62.4) (end 115 61.2635) (width 0.2) (layer "B.Cu") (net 7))
 (segment (start 115 61.2635) (end 116.82 59.4435) (width 0.2) (layer "B.Cu") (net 7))
 (segment (start 118.6 61.4) (end 118.2 61) (width 0.2) (layer "B.Cu") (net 8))
 (segment (start 121.015296 61.873231) (end 120.542065 61.4) (width 0.2) (layer "B.Cu") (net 8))
 (segment (start 118.2 58.2835) (end 116.82 56.9035) (width 0.2) (layer "B.Cu") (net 8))
 (segment (start 120.542065 61.4) (end 118.6 61.4) (width 0.2) (layer "B.Cu") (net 8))
 (segment (start 121.111352 61.873231) (end 121.015296 61.873231) (width 0.2) (layer "B.Cu") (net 8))
 (segment (start 118.2 61) (end 118.2 58.2835) (width 0.2) (layer "B.Cu") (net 8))
 (segment (start 118.2 57) (end 118.2 55.7435) (width 0.2) (layer "B.Cu") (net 9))
 (segment (start 120.549511 59.349511) (end 118.2 57) (width 0.2) (layer "B.Cu") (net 9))
 (segment (start 121.135519 59.349511) (end 120.549511 59.349511) (width 0.2) (layer "B.Cu") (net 9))
 (segment (start 118.2 55.7435) (end 116.82 54.3635) (width 0.2) (layer "B.Cu") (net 9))
 (segment (start 122.810441 54.310441) (end 125.7 57.2) (width 0.5) (layer "B.Cu") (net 11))
 (segment (start 121.135519 54.310441) (end 122.810441 54.310441) (width 0.5) (layer "B.Cu") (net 11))
 (segment (start 124.4 69.6) (end 124.4 71.1) (width 0.5) (layer "B.Cu") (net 16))
 (segment (start 121.8 67) (end 124.4 69.6) (width 0.5) (layer "B.Cu") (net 16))
 (segment (start 104.6 66) (end 105.6 67) (width 0.5) (layer "B.Cu") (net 16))
 (segment (start 111.85 37.8) (end 104.6 45.05) (width 0.5) (layer "B.Cu") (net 16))
 (segment (start 97.435 62.765) (end 95.2 65) (width 0.5) (layer "B.Cu") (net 16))
 (segment (start 104.6 45.05) (end 104.6 64.6) (width 0.5) (layer "B.Cu") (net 16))
 (segment (start 95.2 65) (end 94.61 65) (width 0.5) (layer "B.Cu") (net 16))
 (segment (start 104.6 64.6) (end 104.6 66) (width 0.5) (layer "B.Cu") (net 16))
 (segment (start 111.85 37.8) (end 111.85 40.25) (width 0.5) (layer "B.Cu") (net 16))
 (segment (start 105.6 67) (end 121.8 67) (width 0.5) (layer "B.Cu") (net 16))
 (segment (start 104.6 64.6) (end 99.8775 64.6) (width 0.5) (layer "B.Cu") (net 16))
 (segment (start 99.8775 64.6) (end 98.0425 62.765) (width 0.5) (layer "B.Cu") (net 16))
 (segment (start 111.85 40.25) (end 113.6 42) (width 0.5) (layer "B.Cu") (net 16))
 (segment (start 98.0425 62.765) (end 97.435 62.765) (width 0.5) (layer "B.Cu") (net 16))
 (segment (start 94.61 65) (end 93.31 66.3) (width 0.5) (layer "B.Cu") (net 16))
 (segment (start 100.4 55.7235) (end 101.58 56.9035) (width 0.25) (layer "B.Cu") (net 22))
 (segment (start 97.464481 51.200489) (end 98.416989 51.200489) (width 0.25) (layer "B.Cu") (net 22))
 (segment (start 100.4 53.935608) (end 100.4 55.7235) (width 0.25) (layer "B.Cu") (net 22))
 (segment (start 97.464481 51.200489) (end 97.664881 51.200489) (width 0.25) (layer "B.Cu") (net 22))
 (segment (start 97.664881 51.200489) (end 100.4 53.935608) (width 0.25) (layer "B.Cu") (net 22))
 (segment (start 99.8 54.4) (end 99.8 57.6635) (width 0.25) (layer "B.Cu") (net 21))
 (segment (start 99.079387 53.679387) (end 99.8 54.4) (width 0.25) (layer "B.Cu") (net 21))
 (segment (start 97.464481 53.679387) (end 99.079387 53.679387) (width 0.25) (layer "B.Cu") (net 21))
 (segment (start 99.8 57.6635) (end 101.58 59.4435) (width 0.25) (layer "B.Cu") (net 21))
 (segment (start 97.464481 57.064481) (end 100.4 60) (width 0.25) (layer "B.Cu") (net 20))
 (segment (start 100.7835 61.9835) (end 101.58 61.9835) (width 0.25) (layer "B.Cu") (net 20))
 (segment (start 97.464481 56.239559) (end 97.464481 57.064481) (width 0.25) (layer "B.Cu") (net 20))
 (segment (start 100.4 61.6) (end 100.7835 61.9835) (width 0.25) (layer "B.Cu") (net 20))
 (segment (start 97.464481 56.239559) (end 98.376059 56.239559) (width 0.25) (layer "B.Cu") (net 20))
 (segment (start 100.4 60) (end 100.4 61.6) (width 0.25) (layer "B.Cu") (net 20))
 (segment (start 103 52.9435) (end 101.58 54.3635) (width 0.2) (layer "B.Cu") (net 13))
 (segment (start 101.52 37.7) (end 103 39.18) (width 0.2) (layer "B.Cu") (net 13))
 (segment (start 103 39.18) (end 103 52.9435) (width 0.2) (layer "B.Cu") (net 13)))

